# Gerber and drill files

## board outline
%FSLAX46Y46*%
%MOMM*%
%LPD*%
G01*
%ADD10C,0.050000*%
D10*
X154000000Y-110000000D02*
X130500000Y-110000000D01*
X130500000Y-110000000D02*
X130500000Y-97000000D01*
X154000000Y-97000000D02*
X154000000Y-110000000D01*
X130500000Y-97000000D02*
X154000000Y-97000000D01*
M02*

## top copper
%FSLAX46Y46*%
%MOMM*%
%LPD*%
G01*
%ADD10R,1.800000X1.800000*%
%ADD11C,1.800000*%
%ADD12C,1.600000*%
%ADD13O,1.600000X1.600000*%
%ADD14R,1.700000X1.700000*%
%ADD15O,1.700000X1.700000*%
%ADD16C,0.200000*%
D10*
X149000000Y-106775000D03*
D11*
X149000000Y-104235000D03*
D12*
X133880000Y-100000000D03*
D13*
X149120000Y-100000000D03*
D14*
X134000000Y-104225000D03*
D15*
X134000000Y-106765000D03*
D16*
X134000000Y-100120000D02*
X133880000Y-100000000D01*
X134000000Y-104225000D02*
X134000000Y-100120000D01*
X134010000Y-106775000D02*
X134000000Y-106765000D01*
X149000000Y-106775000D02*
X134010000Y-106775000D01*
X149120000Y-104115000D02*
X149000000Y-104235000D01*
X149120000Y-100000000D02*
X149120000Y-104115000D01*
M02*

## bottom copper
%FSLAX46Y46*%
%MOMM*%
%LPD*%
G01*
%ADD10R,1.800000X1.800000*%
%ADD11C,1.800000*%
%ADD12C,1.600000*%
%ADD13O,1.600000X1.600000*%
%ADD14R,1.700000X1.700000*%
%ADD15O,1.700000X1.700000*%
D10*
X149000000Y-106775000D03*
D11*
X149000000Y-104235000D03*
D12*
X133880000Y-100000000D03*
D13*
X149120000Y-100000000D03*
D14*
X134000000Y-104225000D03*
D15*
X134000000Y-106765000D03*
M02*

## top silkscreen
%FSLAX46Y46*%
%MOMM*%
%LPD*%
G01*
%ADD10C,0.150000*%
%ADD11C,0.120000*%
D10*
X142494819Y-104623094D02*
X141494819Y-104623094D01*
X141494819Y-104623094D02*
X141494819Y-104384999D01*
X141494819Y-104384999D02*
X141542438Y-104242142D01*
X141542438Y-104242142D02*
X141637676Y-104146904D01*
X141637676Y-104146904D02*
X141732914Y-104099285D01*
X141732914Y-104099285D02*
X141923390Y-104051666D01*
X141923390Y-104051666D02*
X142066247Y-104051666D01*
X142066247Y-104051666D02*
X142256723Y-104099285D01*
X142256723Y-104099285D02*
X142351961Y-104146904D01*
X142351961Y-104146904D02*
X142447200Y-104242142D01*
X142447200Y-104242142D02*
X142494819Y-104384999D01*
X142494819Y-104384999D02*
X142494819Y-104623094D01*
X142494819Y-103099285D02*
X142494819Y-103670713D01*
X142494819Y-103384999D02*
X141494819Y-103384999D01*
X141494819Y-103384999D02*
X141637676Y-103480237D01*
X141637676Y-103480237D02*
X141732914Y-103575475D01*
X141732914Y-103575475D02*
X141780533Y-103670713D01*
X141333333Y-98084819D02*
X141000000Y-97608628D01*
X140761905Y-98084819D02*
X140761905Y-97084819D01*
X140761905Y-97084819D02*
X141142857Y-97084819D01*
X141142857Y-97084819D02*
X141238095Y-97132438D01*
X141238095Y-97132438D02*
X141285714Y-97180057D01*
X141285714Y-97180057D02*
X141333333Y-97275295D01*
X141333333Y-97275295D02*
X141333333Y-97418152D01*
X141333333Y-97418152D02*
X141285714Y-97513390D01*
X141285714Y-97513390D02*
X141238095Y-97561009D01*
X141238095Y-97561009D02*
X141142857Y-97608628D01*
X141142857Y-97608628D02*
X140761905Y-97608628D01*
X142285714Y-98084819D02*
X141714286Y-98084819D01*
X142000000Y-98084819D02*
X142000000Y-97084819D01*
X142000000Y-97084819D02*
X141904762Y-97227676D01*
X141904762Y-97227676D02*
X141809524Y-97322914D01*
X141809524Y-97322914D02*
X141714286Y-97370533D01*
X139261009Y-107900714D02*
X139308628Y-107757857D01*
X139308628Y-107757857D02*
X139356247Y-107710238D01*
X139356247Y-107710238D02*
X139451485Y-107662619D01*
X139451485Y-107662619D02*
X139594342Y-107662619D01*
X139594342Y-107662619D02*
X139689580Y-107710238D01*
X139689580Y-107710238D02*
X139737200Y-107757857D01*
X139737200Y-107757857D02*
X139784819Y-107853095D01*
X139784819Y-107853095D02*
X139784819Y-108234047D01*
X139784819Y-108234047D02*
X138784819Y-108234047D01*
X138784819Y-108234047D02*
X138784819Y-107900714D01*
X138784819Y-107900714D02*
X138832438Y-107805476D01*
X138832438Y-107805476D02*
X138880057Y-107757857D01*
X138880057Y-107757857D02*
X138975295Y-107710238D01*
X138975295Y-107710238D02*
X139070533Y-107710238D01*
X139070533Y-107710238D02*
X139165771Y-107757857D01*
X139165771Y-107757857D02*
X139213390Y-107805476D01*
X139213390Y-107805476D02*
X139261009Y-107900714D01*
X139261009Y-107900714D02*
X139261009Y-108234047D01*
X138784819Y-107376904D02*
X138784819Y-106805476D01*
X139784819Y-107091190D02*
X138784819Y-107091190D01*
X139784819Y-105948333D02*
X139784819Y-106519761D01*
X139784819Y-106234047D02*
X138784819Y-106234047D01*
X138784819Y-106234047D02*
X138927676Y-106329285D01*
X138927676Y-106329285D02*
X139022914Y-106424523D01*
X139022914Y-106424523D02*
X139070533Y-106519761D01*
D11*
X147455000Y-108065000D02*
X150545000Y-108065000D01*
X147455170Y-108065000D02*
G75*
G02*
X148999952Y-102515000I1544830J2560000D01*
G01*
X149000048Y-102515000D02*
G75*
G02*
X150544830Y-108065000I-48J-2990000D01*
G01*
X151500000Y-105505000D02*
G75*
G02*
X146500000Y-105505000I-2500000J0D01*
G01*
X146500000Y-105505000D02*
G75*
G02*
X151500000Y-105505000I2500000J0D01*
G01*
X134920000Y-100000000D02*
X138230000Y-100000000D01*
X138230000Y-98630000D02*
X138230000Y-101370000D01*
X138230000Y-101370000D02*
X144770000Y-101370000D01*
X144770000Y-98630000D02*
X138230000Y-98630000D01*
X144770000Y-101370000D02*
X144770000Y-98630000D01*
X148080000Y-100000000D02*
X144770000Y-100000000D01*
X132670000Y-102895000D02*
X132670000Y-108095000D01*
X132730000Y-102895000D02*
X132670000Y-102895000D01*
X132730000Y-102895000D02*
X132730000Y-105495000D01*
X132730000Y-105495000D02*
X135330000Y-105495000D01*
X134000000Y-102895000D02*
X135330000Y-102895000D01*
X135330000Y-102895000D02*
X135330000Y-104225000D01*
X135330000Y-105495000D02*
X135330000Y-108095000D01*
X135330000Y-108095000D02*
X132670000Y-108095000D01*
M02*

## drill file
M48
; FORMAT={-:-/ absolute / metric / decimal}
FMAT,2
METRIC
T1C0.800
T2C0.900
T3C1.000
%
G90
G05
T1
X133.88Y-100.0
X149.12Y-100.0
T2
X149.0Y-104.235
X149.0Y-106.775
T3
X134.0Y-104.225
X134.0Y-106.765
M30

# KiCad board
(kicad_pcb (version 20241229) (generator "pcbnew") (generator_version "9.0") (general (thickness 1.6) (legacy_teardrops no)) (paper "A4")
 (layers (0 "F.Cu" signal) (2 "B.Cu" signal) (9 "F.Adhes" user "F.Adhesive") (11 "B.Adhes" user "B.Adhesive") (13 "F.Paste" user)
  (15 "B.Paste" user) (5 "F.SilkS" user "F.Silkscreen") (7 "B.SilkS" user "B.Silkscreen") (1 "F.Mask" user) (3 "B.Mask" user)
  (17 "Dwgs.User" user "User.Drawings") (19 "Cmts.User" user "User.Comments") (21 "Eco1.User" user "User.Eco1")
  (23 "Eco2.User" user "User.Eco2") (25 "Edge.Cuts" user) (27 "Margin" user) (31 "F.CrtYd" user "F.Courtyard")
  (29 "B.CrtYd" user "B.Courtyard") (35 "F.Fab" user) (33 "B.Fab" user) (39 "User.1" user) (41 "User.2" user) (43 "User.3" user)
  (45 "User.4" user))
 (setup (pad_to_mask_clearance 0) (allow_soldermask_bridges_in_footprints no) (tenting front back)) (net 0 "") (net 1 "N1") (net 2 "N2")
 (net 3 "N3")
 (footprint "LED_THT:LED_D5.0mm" (layer "F.Cu") (at 149 106.775 90)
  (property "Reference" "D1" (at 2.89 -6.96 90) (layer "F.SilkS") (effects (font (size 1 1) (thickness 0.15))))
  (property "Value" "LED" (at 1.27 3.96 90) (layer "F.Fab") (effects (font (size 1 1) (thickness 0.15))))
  (fp_line (start -1.29 -1.545) (end -1.29 1.545) (stroke (width 0.12) (type solid)) (layer "F.SilkS"))
  (fp_arc (start -1.29 -1.54483) (mid 2.071756 -2.880501) (end 4.26 -0.000048) (stroke (width 0.12) (type solid)) (layer "F.SilkS"))
  (fp_arc (start 4.26 0.000048) (mid 2.071756 2.880501) (end -1.29 1.54483) (stroke (width 0.12) (type solid)) (layer "F.SilkS"))
  (fp_circle (center 1.27 0) (end 3.77 0) (stroke (width 0.12) (type solid)) (fill no) (layer "F.SilkS"))
  (pad "1" thru_hole rect (at 0 0 90) (size 1.8 1.8) (drill 0.9) (layers "*.Cu" "*.Mask") (remove_unused_layers no) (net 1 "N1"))
  (pad "2" thru_hole circle (at 2.54 0 90) (size 1.8 1.8) (drill 0.9) (layers "*.Cu" "*.Mask") (remove_unused_layers no) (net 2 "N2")))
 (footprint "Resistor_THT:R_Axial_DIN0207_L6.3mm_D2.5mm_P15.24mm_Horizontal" (layer "F.Cu") (at 133.88 100)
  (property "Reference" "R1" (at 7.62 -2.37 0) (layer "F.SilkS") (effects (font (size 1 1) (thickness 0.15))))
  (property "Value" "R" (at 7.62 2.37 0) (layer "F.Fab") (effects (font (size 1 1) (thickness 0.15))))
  (fp_line (start 1.04 0) (end 4.35 0) (stroke (width 0.12) (type solid)) (layer "F.SilkS"))
  (fp_line (start 4.35 -1.37) (end 4.35 1.37) (stroke (width 0.12) (type solid)) (layer "F.SilkS"))
  (fp_line (start 4.35 1.37) (end 10.89 1.37) (stroke (width 0.12) (type solid)) (layer "F.SilkS"))
  (fp_line (start 10.89 -1.37) (end 4.35 -1.37) (stroke (width 0.12) (type solid)) (layer "F.SilkS"))
  (fp_line (start 10.89 1.37) (end 10.89 -1.37) (stroke (width 0.12) (type solid)) (layer "F.SilkS"))
  (fp_line (start 14.2 0) (end 10.89 0) (stroke (width 0.12) (type solid)) (layer "F.SilkS"))
  (pad "1" thru_hole circle (at 0 0) (size 1.6 1.6) (drill 0.8) (layers "*.Cu" "*.Mask") (remove_unused_layers no) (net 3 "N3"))
  (pad "2" thru_hole oval (at 15.24 0) (size 1.6 1.6) (drill 0.8) (layers "*.Cu" "*.Mask") (remove_unused_layers no) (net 2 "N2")))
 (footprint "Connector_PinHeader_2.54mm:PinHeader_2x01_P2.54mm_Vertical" (layer "F.Cu") (at 134 104.225 -90)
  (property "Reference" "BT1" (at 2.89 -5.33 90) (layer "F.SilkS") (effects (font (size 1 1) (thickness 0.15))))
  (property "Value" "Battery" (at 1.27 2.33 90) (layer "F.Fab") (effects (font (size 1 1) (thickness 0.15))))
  (fp_line (start -1.33 1.33) (end 3.87 1.33) (stroke (width 0.12) (type solid)) (layer "F.SilkS"))
  (fp_line (start -1.33 1.27) (end -1.33 1.33) (stroke (width 0.12) (type solid)) (layer "F.SilkS"))
  (fp_line (start -1.33 1.27) (end 1.27 1.27) (stroke (width 0.12) (type solid)) (layer "F.SilkS"))
  (fp_line (start 1.27 1.27) (end 1.27 -1.33) (stroke (width 0.12) (type solid)) (layer "F.SilkS"))
  (fp_line (start -1.33 0) (end -1.33 -1.33) (stroke (width 0.12) (type solid)) (layer "F.SilkS"))
  (fp_line (start -1.33 -1.33) (end 0 -1.33) (stroke (width 0.12) (type solid)) (layer "F.SilkS"))
  (fp_line (start 1.27 -1.33) (end 3.87 -1.33) (stroke (width 0.12) (type solid)) (layer "F.SilkS"))
  (fp_line (start 3.87 -1.33) (end 3.87 1.33) (stroke (width 0.12) (type solid)) (layer "F.SilkS"))
  (pad "1" thru_hole rect (at 0 0 270) (size 1.7 1.7) (drill 1) (layers "*.Cu" "*.Mask") (remove_unused_layers no) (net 3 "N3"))
  (pad "2" thru_hole oval (at 2.54 0 270) (size 1.7 1.7) (drill 1) (layers "*.Cu" "*.Mask") (remove_unused_layers no) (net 1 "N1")))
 (gr_line (start 154 110) (end 130.5 110) (stroke (width 0.05) (type default)) (layer "Edge.Cuts"))
 (gr_line (start 130.5 110) (end 130.5 97) (stroke (width 0.05) (type default)) (layer "Edge.Cuts"))
 (gr_line (start 154 97) (end 154 110) (stroke (width 0.05) (type default)) (layer "Edge.Cuts"))
 (gr_line (start 130.5 97) (end 154 97) (stroke (width 0.05) (type default)) (layer "Edge.Cuts"))
 (segment (start 134 100.12) (end 133.88 100) (width 0.2) (layer "F.Cu") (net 3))
 (segment (start 134 104.225) (end 134 100.12) (width 0.2) (layer "F.Cu") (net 3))
 (segment (start 134.01 106.775) (end 134 106.765) (width 0.2) (layer "F.Cu") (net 1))
 (segment (start 149 106.775) (end 134.01 106.775) (width 0.2) (layer "F.Cu") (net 1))
 (segment (start 149.12 104.115) (end 149 104.235) (width 0.2) (layer "F.Cu") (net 2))
 (segment (start 149.12 100) (end 149.12 104.115) (width 0.2) (layer "F.Cu") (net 2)))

